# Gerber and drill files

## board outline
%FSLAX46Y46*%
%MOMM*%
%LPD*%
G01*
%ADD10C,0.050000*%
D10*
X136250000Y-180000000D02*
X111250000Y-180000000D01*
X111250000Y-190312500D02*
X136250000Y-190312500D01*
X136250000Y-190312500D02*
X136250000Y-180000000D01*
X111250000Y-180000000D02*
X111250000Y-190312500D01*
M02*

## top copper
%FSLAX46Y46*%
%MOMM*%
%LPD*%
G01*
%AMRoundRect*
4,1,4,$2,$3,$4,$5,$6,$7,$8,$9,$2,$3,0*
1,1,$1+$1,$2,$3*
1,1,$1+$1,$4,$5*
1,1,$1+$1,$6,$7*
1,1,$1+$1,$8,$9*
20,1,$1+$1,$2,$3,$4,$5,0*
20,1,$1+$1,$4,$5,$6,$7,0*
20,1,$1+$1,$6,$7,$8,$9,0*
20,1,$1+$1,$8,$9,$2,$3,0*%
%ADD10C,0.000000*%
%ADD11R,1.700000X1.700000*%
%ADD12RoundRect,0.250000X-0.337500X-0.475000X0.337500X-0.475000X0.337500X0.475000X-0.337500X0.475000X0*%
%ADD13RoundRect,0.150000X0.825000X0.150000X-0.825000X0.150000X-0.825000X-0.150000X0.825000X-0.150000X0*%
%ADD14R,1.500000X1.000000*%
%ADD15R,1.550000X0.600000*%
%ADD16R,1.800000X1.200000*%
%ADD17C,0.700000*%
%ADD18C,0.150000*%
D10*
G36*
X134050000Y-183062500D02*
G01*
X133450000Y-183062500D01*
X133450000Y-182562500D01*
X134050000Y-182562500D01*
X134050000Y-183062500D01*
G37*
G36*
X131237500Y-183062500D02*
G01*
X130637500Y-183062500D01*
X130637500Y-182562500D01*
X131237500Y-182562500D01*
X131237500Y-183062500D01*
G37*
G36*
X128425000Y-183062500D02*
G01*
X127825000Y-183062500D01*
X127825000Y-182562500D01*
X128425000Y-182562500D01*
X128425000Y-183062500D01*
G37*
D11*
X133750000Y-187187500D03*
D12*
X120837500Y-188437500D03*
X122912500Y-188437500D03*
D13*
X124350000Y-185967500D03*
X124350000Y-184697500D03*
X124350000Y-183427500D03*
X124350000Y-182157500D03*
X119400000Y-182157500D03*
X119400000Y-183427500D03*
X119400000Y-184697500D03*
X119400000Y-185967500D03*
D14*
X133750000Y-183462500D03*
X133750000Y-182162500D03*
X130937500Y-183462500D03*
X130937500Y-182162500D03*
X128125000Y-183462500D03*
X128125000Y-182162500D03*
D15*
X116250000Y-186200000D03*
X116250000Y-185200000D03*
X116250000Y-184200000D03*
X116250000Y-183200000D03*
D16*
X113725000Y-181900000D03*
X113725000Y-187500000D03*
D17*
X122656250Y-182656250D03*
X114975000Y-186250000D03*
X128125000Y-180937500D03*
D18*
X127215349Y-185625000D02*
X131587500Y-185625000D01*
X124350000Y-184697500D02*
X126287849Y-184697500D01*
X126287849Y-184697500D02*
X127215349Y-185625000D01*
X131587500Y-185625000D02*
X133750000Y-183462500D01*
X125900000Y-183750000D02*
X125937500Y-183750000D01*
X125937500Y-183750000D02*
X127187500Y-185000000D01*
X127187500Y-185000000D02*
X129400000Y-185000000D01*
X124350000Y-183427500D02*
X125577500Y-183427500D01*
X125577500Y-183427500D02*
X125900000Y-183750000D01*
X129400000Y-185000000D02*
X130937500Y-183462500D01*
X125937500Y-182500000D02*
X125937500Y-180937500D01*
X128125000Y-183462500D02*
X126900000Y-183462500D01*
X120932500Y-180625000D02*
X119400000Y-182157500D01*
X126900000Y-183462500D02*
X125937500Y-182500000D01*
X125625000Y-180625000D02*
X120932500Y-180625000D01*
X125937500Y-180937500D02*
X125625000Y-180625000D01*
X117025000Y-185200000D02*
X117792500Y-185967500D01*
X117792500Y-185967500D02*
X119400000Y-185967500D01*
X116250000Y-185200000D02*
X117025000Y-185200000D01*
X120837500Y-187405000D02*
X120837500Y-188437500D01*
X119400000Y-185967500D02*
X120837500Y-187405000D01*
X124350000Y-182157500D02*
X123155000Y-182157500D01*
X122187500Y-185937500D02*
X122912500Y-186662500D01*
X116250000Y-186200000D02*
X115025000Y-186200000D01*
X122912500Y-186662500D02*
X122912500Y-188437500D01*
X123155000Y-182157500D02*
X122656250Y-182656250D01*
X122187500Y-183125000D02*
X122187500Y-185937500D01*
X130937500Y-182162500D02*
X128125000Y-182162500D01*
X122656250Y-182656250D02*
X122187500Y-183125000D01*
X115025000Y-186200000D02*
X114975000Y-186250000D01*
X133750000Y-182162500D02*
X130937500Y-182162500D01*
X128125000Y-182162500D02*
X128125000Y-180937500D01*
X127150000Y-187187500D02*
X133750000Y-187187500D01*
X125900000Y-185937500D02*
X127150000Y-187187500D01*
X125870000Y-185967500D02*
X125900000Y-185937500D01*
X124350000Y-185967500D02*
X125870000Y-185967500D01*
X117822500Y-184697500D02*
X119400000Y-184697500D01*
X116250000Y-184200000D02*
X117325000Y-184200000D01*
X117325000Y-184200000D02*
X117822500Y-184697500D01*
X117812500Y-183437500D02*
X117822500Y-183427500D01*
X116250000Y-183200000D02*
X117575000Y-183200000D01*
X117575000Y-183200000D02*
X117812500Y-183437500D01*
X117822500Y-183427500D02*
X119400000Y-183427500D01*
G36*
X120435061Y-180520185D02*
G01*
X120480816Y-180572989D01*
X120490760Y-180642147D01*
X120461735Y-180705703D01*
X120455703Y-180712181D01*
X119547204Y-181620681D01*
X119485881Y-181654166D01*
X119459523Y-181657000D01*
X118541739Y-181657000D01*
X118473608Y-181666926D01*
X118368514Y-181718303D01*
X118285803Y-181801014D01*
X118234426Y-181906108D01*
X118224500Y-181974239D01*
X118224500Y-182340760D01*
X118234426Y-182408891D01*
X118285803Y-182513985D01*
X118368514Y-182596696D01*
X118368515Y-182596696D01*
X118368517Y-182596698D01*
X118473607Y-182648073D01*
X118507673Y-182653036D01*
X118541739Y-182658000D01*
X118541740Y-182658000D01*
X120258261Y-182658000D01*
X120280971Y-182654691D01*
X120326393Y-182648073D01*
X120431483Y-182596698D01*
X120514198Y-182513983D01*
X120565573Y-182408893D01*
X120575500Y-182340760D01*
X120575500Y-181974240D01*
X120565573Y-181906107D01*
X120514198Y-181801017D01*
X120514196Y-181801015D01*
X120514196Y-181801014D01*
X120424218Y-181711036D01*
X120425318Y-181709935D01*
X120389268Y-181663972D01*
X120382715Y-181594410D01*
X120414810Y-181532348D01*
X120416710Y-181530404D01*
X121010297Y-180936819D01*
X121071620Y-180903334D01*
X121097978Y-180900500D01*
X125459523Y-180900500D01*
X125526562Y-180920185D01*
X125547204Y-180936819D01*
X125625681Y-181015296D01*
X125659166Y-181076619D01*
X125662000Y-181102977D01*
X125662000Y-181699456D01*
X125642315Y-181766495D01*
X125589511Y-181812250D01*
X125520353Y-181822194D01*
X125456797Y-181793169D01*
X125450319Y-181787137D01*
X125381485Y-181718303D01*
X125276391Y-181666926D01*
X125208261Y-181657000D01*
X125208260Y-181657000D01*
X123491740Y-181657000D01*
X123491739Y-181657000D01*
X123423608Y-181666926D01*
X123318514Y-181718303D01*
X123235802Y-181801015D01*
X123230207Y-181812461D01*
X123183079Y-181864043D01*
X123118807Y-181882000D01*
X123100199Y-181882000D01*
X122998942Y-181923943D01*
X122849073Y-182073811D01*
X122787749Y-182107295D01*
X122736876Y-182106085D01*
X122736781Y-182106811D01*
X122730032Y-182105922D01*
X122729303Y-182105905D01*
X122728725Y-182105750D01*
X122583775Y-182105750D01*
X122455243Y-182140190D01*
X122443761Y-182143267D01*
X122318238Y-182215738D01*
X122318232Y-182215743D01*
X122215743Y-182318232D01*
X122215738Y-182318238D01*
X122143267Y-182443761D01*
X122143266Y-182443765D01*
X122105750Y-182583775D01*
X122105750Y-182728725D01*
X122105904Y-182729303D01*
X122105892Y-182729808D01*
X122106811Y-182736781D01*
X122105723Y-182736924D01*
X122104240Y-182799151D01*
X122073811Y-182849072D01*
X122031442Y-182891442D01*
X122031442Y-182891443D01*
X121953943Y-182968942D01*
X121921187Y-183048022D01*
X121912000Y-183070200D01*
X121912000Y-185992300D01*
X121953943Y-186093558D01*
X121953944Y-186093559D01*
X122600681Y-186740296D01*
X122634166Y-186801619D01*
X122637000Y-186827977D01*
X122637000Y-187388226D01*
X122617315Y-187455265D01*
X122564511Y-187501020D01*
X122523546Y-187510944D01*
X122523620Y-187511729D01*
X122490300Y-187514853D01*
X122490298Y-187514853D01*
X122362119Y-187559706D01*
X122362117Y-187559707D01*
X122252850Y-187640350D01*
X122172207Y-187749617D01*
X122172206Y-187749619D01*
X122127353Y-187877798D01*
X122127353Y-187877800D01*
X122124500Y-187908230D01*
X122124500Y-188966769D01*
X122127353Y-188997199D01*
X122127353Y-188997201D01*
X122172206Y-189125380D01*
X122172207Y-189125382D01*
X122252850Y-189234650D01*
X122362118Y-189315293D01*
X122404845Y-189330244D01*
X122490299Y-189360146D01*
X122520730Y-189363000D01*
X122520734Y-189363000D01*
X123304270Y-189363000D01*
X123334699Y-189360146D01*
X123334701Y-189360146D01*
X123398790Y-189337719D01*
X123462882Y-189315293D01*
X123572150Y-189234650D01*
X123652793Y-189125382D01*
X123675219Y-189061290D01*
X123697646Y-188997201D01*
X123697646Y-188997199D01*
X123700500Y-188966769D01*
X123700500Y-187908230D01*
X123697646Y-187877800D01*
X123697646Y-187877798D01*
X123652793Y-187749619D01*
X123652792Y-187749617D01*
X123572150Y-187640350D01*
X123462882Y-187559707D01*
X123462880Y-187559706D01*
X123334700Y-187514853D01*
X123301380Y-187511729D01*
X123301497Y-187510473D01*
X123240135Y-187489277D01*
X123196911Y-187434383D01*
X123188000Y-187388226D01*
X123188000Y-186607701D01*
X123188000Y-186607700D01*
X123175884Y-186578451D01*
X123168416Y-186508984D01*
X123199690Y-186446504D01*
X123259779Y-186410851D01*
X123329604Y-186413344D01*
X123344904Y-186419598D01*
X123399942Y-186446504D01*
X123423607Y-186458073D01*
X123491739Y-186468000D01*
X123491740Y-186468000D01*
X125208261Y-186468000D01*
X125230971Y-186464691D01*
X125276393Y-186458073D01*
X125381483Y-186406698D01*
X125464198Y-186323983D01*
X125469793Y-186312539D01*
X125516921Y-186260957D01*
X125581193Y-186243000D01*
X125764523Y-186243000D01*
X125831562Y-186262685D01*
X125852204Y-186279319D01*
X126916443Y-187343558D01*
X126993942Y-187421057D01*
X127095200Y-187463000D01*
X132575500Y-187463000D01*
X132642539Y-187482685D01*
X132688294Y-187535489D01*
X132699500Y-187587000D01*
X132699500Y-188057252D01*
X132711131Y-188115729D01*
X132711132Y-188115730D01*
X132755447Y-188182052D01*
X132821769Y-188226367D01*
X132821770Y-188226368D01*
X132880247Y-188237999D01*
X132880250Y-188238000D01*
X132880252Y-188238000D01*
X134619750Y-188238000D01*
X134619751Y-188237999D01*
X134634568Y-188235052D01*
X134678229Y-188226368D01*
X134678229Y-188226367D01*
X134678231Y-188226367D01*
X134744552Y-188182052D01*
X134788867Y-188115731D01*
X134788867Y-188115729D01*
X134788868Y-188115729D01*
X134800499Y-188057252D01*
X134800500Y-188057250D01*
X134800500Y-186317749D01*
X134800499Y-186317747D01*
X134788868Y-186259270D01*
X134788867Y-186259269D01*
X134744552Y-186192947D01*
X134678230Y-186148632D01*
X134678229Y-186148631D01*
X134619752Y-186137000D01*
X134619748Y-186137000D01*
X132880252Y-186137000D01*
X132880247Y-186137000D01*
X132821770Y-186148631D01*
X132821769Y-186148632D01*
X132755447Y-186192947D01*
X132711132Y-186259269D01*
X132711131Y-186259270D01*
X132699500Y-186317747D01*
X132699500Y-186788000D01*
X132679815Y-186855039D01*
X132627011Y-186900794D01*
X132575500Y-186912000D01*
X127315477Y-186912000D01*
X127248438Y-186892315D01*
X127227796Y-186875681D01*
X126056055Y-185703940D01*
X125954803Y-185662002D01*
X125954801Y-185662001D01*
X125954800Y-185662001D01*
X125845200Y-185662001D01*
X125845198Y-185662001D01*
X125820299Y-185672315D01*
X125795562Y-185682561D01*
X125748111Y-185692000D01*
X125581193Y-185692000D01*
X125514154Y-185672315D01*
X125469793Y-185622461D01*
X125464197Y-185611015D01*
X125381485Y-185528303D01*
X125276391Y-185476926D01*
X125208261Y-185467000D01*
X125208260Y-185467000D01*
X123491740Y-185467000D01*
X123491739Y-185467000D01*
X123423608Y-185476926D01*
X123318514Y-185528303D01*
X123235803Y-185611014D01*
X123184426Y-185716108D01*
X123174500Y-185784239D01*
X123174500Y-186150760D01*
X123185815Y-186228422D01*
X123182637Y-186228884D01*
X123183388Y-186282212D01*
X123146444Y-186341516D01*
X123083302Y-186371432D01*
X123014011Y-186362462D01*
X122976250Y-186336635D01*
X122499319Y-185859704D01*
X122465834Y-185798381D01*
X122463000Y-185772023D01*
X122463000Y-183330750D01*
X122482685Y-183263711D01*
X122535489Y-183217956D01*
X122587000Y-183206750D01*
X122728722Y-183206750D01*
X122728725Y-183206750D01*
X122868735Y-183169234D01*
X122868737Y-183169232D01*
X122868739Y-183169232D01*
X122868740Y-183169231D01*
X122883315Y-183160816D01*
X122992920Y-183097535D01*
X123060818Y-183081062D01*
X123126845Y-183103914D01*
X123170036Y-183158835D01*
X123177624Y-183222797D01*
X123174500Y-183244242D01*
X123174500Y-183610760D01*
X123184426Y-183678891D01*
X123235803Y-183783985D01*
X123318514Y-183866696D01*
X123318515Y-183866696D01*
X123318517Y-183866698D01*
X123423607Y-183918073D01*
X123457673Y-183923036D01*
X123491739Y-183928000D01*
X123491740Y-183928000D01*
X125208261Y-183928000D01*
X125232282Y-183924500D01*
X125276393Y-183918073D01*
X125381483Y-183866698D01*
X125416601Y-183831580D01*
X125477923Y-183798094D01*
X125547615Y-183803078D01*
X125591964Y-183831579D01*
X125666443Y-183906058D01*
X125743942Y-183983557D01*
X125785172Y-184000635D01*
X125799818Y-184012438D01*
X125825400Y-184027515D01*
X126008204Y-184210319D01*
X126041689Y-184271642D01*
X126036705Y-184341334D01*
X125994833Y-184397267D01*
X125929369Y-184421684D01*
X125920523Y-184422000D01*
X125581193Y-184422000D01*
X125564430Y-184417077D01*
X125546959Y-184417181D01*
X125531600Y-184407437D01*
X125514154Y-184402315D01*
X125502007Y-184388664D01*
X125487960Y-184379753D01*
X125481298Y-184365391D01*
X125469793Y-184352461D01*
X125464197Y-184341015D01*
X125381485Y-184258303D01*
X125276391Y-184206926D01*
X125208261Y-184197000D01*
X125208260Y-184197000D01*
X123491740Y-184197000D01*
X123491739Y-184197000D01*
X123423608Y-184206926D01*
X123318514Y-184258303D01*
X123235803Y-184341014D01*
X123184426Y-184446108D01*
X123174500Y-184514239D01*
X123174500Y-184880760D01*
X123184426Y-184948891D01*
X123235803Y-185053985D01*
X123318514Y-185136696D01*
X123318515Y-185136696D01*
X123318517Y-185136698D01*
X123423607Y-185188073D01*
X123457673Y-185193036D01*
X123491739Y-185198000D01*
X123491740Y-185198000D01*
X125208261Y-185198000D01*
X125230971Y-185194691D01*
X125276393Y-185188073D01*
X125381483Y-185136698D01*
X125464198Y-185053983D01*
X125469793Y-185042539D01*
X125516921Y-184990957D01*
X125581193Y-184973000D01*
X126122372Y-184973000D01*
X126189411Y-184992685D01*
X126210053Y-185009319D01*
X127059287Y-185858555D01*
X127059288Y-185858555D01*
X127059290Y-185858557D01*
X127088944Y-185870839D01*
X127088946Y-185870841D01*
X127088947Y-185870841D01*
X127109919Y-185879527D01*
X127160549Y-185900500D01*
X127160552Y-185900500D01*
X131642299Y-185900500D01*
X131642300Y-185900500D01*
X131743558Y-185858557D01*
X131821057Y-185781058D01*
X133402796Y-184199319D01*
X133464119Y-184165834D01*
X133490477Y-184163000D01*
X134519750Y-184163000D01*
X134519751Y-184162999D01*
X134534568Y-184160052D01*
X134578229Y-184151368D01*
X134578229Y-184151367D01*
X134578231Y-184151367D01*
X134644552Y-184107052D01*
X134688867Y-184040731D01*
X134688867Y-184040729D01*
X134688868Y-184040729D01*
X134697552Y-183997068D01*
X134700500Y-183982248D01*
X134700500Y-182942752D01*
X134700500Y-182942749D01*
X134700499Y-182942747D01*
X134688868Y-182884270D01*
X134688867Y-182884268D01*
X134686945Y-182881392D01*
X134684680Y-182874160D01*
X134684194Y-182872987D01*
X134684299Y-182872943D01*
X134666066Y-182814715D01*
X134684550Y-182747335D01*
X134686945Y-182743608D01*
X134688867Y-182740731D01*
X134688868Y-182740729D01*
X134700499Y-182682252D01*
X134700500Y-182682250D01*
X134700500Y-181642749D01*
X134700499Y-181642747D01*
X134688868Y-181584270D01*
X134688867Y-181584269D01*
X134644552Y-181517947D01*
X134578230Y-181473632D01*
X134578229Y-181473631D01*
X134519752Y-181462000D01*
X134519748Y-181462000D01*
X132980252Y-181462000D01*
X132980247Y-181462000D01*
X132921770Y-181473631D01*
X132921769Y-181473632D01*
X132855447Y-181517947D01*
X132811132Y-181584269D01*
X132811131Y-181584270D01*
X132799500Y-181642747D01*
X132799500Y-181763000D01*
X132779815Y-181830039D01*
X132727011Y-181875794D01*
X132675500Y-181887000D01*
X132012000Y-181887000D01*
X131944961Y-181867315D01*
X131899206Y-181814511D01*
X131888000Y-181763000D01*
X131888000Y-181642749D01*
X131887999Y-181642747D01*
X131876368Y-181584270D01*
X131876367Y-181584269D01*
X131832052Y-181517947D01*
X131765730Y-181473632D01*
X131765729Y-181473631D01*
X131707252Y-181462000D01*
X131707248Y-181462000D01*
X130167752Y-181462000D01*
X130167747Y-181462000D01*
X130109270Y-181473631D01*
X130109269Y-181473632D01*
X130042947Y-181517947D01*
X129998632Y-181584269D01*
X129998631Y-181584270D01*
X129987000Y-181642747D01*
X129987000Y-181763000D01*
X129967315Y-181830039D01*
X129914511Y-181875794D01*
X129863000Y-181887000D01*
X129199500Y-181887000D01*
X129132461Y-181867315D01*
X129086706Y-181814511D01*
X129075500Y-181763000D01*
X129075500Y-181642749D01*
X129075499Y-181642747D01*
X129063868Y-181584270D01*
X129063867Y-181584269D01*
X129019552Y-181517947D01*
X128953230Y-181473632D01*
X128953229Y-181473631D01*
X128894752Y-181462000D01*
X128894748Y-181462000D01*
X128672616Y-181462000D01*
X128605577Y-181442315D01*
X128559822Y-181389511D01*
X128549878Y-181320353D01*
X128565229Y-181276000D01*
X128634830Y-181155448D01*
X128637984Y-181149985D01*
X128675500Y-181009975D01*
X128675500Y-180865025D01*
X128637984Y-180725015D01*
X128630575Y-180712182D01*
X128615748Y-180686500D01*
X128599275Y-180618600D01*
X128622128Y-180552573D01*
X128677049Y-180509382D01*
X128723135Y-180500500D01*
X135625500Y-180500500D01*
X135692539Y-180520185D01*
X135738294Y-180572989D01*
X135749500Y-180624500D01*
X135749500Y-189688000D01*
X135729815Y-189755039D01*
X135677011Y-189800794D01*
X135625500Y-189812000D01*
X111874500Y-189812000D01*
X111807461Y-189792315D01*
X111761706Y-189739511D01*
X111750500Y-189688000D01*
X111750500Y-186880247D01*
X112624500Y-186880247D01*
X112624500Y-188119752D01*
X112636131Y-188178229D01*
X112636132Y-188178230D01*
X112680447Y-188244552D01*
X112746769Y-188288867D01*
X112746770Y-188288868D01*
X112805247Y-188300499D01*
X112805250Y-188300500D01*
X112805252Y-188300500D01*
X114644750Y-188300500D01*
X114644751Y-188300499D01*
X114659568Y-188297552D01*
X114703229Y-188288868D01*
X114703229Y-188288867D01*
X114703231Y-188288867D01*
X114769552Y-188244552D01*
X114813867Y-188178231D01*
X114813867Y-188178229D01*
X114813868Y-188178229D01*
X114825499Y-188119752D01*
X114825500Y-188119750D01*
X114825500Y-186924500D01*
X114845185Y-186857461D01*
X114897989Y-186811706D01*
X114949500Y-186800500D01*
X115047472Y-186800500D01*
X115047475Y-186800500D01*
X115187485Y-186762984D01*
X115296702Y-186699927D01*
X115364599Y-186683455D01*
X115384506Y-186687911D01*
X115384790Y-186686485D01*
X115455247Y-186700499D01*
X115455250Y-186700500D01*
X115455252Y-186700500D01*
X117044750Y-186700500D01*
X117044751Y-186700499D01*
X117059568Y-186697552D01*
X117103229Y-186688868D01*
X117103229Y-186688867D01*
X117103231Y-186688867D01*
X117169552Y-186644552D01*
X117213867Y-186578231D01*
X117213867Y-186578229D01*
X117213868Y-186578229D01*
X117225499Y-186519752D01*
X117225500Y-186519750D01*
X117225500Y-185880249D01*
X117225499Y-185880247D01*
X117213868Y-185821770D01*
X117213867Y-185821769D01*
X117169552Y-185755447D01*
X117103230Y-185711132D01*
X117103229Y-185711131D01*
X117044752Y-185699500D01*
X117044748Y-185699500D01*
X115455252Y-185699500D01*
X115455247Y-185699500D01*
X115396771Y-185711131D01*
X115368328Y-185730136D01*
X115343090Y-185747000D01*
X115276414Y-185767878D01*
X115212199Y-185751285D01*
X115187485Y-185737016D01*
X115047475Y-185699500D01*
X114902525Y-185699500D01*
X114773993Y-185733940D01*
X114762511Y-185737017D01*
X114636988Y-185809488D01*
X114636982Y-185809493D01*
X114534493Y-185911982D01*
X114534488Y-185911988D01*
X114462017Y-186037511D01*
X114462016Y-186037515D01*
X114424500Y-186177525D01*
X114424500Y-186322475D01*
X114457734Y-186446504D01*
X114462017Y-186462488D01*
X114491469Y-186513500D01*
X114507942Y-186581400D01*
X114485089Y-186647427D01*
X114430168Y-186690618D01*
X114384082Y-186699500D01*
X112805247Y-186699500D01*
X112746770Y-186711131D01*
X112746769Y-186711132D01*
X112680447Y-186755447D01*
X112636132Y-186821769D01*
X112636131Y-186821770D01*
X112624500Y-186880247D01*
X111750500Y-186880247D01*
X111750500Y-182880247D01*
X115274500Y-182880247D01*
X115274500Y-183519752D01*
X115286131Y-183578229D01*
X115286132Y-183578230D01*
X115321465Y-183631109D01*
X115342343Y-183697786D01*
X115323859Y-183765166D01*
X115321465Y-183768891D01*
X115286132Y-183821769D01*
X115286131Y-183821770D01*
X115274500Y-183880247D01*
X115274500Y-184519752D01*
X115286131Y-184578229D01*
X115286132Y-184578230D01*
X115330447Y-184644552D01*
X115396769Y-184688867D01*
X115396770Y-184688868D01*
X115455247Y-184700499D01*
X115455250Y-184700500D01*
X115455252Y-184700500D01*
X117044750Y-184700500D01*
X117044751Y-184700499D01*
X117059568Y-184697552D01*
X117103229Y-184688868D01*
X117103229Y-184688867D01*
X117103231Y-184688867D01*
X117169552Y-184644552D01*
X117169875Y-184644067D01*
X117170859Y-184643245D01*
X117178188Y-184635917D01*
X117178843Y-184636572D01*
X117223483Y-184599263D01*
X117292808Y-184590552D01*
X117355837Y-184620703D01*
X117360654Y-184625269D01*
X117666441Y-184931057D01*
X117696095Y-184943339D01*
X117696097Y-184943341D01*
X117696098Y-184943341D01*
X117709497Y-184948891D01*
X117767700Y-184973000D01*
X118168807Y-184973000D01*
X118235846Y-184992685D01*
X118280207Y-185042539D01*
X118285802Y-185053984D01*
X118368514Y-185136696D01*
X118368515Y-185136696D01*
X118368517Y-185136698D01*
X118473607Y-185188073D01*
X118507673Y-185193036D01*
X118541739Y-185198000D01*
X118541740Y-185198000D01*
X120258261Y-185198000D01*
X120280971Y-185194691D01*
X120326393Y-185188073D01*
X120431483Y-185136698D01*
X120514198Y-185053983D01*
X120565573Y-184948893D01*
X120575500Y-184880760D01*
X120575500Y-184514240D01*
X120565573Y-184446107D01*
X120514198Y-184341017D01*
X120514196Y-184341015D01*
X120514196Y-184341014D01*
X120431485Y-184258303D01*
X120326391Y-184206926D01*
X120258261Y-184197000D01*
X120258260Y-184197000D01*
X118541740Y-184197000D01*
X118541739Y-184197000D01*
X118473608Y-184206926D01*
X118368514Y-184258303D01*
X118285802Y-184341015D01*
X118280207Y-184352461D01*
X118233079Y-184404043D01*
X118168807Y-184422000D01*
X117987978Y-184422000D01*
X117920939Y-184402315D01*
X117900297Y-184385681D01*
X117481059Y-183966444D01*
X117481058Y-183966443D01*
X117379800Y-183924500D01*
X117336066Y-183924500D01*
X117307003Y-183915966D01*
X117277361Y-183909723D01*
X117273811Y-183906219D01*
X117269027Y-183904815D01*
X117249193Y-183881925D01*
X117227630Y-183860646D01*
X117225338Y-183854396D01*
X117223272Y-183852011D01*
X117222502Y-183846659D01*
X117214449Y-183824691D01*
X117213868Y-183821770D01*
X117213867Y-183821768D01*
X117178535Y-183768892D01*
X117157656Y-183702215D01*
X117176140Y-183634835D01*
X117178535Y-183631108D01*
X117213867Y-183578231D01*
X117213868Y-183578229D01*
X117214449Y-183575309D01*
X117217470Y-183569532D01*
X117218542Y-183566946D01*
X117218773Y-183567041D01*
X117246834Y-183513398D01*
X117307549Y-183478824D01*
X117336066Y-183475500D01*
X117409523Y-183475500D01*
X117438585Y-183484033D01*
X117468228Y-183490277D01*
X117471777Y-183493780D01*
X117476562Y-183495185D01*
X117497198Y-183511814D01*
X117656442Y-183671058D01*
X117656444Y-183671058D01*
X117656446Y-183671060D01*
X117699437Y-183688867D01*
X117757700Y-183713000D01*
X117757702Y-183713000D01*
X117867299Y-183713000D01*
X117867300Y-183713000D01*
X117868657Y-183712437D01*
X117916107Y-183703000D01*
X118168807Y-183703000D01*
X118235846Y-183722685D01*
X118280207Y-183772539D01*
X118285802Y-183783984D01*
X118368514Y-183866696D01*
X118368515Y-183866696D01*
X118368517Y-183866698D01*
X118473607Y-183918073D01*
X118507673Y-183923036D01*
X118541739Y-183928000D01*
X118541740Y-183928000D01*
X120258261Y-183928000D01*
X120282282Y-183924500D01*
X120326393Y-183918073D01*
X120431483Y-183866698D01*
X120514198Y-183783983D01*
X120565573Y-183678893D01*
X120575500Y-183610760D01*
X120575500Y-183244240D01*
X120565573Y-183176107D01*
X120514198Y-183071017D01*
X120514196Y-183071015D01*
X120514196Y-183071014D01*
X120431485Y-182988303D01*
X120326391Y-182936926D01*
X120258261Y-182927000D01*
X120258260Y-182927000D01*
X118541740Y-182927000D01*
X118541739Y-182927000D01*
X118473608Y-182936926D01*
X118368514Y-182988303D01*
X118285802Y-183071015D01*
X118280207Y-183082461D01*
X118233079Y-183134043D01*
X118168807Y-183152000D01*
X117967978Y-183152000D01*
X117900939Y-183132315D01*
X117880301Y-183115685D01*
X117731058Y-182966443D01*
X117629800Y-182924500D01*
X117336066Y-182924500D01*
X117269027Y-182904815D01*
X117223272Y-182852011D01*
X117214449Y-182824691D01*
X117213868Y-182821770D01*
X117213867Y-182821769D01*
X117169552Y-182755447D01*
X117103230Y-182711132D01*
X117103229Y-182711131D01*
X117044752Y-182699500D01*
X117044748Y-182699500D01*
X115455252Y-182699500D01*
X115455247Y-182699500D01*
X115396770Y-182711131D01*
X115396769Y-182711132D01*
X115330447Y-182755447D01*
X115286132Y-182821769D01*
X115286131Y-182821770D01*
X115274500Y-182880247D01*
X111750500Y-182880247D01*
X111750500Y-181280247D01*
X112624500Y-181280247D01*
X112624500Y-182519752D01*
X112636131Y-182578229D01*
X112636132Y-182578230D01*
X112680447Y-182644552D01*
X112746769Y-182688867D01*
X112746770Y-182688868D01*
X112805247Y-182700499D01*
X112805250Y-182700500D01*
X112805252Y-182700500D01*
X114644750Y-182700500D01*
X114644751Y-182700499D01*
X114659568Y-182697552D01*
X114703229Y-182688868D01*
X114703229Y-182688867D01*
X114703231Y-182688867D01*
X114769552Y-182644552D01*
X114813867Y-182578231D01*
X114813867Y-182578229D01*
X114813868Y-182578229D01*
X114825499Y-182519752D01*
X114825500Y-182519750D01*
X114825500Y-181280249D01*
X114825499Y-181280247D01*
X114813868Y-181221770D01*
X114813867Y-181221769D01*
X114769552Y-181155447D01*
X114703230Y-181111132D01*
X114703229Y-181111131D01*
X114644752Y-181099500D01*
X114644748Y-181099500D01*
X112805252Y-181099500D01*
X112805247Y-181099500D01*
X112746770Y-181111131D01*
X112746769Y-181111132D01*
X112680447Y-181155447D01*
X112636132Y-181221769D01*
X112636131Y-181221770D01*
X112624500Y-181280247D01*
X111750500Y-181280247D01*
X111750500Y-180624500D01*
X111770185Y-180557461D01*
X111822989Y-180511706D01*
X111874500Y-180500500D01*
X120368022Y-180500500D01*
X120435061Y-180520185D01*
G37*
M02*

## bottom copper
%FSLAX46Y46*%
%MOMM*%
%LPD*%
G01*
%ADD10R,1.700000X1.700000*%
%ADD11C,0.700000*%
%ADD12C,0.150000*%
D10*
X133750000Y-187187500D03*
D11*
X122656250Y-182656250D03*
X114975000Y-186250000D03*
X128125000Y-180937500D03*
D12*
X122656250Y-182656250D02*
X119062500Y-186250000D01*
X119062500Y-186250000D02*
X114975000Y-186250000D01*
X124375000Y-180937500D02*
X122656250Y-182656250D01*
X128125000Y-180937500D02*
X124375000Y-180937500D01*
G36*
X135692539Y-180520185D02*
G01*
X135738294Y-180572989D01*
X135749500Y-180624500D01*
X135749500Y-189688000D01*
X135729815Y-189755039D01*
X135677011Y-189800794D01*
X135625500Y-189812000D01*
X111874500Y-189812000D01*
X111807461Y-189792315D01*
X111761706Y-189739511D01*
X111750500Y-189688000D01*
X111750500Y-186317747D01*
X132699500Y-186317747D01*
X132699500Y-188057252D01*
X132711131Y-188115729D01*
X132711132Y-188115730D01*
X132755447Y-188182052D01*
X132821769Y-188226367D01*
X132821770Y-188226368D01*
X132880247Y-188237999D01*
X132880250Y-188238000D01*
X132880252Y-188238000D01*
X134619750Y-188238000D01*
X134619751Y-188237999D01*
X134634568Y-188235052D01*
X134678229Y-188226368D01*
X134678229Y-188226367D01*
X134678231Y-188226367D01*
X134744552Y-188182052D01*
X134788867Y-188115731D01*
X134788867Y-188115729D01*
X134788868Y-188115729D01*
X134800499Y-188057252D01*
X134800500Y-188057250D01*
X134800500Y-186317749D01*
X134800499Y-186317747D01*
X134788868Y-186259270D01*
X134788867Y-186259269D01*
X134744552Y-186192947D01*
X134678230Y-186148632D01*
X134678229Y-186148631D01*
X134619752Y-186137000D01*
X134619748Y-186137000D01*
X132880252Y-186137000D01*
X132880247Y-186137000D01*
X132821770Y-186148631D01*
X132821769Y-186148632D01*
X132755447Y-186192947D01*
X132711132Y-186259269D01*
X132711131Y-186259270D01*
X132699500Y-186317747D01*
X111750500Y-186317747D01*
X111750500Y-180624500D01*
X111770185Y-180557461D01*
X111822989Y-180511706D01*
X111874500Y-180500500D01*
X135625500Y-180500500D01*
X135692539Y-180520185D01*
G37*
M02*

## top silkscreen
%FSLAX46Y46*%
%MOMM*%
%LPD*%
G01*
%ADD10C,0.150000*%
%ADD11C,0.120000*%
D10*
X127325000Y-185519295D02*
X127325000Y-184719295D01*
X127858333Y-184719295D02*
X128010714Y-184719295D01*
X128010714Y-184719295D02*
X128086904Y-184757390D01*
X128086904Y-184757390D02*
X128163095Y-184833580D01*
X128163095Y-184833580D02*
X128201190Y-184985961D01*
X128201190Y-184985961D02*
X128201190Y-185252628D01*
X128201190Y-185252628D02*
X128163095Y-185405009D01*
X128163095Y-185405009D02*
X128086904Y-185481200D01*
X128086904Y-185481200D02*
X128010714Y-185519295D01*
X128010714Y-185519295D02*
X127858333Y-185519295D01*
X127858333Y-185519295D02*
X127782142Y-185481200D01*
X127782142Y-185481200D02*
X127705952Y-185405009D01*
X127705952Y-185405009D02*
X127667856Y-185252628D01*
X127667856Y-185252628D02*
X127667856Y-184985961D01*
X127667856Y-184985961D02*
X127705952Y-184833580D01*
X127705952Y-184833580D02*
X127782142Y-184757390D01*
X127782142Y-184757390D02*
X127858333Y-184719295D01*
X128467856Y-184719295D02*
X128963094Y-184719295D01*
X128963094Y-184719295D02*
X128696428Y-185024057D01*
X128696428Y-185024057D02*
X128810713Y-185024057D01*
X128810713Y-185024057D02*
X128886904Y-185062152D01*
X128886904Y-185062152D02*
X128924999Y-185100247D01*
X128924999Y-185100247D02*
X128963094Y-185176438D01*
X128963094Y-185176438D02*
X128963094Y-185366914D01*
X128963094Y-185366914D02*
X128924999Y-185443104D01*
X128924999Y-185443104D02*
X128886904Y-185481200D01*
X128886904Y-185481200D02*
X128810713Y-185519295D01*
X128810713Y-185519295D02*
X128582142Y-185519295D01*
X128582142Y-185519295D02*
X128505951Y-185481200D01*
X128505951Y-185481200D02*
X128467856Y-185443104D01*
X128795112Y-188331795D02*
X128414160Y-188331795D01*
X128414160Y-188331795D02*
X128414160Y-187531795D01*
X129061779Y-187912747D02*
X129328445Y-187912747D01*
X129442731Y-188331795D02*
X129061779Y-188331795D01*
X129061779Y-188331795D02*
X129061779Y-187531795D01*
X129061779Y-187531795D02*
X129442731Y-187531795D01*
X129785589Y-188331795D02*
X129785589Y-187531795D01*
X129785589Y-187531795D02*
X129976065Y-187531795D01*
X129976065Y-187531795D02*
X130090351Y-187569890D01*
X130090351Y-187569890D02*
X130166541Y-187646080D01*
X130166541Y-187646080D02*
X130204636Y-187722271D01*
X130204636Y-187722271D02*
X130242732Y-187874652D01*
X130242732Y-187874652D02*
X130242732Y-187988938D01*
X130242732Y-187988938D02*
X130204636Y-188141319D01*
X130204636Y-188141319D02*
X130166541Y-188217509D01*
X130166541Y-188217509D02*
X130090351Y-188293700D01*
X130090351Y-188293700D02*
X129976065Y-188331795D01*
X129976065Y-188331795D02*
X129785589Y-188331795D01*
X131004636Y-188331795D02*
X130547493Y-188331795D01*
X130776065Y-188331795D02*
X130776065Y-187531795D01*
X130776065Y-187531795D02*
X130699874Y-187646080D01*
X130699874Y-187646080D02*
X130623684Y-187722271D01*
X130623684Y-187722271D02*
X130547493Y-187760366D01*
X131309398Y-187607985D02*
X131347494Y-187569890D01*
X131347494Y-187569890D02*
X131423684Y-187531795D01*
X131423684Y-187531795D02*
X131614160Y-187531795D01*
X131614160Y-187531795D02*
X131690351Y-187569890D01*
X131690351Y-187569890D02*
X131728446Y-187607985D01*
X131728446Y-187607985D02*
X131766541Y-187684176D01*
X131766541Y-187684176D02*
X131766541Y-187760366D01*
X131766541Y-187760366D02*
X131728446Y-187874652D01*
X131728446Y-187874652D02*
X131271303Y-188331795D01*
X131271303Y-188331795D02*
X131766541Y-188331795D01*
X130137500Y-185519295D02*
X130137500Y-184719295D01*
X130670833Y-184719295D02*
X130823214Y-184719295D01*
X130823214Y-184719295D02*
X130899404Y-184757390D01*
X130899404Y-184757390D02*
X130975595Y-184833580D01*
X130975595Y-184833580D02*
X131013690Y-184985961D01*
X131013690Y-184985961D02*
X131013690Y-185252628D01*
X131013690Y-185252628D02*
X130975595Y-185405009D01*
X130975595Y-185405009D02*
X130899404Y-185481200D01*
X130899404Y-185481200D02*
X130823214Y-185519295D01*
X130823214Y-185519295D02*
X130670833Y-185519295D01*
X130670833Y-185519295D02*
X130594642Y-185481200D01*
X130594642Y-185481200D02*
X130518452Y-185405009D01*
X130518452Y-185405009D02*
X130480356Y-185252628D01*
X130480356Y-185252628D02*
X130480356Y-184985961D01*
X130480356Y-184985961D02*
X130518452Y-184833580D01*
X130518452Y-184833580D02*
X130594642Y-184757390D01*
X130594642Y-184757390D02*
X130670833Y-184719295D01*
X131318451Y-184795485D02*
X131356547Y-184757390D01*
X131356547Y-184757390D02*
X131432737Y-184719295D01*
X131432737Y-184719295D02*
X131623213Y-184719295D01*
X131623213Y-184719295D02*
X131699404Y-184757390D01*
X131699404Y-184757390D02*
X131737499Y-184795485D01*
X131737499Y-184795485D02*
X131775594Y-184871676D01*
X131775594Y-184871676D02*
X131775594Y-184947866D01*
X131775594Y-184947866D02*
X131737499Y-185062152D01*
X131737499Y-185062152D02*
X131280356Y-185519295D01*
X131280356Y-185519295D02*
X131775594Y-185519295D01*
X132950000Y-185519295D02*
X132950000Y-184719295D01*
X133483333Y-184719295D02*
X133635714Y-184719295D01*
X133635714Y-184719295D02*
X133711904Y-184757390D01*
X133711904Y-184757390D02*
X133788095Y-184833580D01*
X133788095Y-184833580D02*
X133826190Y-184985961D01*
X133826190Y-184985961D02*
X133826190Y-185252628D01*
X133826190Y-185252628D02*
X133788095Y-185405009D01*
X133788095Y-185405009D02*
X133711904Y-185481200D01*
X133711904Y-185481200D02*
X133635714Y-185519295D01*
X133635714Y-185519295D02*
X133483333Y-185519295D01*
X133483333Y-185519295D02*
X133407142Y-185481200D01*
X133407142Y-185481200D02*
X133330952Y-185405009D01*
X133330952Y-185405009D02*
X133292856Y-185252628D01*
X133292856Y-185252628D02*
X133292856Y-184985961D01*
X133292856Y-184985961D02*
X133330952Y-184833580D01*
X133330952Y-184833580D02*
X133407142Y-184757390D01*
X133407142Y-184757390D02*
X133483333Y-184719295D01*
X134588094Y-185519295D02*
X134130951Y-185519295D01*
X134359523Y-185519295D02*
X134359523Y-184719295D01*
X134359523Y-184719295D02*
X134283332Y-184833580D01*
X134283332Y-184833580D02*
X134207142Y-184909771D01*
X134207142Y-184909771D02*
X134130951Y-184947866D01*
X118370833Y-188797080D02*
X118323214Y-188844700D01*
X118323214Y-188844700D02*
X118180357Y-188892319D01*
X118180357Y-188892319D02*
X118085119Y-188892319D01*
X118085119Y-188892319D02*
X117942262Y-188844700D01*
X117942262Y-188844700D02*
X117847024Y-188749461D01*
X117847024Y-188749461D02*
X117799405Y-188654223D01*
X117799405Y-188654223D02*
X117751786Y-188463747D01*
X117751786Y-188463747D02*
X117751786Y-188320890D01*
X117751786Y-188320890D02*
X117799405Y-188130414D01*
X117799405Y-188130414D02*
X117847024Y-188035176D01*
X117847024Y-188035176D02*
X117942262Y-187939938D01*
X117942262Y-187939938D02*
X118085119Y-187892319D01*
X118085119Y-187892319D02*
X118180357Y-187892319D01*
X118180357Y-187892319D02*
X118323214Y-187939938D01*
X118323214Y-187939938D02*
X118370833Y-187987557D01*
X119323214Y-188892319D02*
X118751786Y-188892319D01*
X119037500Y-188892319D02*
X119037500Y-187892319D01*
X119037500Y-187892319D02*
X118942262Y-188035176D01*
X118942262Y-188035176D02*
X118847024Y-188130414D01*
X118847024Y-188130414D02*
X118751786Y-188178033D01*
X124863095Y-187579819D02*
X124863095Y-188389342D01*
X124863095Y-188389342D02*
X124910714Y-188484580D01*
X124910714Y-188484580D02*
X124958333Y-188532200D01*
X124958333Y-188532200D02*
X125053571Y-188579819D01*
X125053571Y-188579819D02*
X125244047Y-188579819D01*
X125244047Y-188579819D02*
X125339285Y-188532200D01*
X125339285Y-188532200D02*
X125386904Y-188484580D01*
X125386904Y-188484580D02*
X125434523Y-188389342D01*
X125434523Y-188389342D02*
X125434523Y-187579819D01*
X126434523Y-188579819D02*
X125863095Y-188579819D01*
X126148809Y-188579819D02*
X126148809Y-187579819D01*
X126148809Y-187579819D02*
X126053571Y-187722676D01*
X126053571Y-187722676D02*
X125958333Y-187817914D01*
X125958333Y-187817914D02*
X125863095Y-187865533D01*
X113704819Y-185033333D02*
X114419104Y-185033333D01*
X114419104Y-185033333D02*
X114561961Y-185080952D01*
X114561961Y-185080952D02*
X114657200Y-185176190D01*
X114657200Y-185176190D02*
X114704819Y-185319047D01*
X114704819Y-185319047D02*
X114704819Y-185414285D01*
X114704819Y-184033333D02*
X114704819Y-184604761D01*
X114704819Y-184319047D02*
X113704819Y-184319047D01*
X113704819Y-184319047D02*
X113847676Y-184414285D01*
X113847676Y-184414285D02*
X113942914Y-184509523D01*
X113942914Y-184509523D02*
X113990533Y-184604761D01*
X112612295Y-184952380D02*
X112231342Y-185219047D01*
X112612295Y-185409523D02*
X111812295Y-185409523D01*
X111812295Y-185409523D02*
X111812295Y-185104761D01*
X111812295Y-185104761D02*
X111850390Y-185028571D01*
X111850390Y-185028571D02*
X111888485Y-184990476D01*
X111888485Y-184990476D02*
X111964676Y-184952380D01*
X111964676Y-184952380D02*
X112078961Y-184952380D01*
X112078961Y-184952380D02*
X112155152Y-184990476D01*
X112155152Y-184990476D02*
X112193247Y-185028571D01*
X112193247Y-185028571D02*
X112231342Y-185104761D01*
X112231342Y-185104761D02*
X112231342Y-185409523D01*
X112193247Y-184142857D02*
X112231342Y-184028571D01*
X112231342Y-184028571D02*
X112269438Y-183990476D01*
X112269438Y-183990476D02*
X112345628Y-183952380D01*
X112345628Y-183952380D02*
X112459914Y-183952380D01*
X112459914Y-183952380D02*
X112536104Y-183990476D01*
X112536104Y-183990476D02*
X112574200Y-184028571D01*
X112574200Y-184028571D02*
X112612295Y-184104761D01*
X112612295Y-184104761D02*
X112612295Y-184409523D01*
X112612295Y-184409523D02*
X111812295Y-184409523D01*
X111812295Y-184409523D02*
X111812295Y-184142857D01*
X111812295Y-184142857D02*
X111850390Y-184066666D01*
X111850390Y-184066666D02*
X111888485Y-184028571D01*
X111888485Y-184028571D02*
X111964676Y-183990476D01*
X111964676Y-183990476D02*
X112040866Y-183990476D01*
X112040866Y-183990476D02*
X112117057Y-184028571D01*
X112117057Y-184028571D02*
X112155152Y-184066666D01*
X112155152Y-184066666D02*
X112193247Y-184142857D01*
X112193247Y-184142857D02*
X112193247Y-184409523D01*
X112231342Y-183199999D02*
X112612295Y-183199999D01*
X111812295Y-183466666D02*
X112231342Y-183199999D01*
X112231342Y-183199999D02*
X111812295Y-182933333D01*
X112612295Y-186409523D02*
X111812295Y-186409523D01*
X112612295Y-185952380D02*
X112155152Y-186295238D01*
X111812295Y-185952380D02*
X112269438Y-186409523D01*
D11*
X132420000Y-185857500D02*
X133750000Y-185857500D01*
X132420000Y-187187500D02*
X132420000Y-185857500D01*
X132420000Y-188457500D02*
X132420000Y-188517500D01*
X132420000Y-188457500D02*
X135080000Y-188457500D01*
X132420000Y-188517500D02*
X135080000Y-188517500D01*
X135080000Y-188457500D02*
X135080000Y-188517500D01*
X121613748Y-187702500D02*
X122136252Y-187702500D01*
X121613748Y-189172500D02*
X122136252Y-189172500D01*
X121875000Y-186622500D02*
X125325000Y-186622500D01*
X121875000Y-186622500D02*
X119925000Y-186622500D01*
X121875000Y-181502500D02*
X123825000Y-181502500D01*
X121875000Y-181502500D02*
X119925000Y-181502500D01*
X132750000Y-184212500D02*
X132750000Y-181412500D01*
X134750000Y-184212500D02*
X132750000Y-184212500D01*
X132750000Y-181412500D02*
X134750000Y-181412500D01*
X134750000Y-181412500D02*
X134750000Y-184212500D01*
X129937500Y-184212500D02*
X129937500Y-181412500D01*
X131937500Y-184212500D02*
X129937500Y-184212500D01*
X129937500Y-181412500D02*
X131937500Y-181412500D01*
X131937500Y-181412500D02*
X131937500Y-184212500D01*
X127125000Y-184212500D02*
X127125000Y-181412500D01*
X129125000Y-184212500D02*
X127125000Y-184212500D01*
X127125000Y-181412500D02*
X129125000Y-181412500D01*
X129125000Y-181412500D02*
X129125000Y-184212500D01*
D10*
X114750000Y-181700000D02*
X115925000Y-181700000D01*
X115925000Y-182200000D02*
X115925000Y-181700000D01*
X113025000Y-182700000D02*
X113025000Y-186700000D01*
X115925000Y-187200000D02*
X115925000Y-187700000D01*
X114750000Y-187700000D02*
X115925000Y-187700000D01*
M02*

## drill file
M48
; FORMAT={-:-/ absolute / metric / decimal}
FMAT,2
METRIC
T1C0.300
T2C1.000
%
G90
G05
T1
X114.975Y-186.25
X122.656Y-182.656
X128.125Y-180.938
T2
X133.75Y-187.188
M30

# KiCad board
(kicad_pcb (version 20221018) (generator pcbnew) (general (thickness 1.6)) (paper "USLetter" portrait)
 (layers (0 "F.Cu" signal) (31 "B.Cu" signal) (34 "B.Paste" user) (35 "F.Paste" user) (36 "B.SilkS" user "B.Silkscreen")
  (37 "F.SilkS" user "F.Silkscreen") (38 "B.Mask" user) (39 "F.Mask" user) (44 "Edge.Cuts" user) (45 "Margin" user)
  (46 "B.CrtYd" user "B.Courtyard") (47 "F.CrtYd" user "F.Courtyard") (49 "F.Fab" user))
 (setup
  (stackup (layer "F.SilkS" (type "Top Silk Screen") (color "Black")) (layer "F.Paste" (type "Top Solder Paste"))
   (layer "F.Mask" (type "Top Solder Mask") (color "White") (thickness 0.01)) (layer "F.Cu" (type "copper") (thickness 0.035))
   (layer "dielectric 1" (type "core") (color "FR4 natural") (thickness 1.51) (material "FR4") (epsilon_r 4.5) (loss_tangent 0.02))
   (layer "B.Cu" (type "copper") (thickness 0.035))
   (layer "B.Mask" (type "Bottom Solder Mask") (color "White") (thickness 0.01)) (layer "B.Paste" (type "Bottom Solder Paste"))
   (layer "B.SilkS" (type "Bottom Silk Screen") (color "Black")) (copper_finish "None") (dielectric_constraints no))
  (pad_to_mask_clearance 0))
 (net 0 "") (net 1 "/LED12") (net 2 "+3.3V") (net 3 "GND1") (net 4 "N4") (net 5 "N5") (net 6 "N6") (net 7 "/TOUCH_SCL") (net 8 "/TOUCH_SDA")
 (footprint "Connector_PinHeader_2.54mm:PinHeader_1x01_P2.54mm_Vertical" (layer "F.Cu") (at 133.75 187.1875)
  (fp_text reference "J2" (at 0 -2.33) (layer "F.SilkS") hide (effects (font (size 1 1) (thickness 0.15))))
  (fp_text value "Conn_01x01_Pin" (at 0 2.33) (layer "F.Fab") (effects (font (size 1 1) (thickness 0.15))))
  (fp_line (start -1.33 -1.33) (end 0 -1.33) (stroke (width 0.12) (type solid)) (layer "F.SilkS"))
  (fp_line (start -1.33 0) (end -1.33 -1.33) (stroke (width 0.12) (type solid)) (layer "F.SilkS"))
  (fp_line (start -1.33 1.27) (end -1.33 1.33) (stroke (width 0.12) (type solid)) (layer "F.SilkS"))
  (fp_line (start -1.33 1.27) (end 1.33 1.27) (stroke (width 0.12) (type solid)) (layer "F.SilkS"))
  (fp_line (start -1.33 1.33) (end 1.33 1.33) (stroke (width 0.12) (type solid)) (layer "F.SilkS"))
  (fp_line (start 1.33 1.27) (end 1.33 1.33) (stroke (width 0.12) (type solid)) (layer "F.SilkS"))
  (pad "1" thru_hole rect (at 0 0) (size 1.7 1.7) (drill 1) (layers "*.Cu" "*.Mask") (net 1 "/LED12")))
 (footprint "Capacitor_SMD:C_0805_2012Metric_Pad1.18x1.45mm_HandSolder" (layer "F.Cu") (at 121.875 188.4375)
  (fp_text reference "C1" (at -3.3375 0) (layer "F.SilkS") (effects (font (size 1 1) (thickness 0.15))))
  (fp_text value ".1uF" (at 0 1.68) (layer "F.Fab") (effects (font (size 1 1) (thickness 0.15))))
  (fp_line (start -0.261252 -0.735) (end 0.261252 -0.735) (stroke (width 0.12) (type solid)) (layer "F.SilkS"))
  (fp_line (start -0.261252 0.735) (end 0.261252 0.735) (stroke (width 0.12) (type solid)) (layer "F.SilkS"))
  (pad "1" smd roundrect (at -1.0375 0) (size 1.175 1.45) (layers "F.Cu" "F.Paste" "F.Mask") (roundrect_rratio 0.2127659574) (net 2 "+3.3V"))
  (pad "2" smd roundrect (at 1.0375 0) (size 1.175 1.45) (layers "F.Cu" "F.Paste" "F.Mask") (roundrect_rratio 0.2127659574) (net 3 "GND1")))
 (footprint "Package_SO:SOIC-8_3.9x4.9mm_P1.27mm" (layer "F.Cu") (at 121.875 184.0625 180)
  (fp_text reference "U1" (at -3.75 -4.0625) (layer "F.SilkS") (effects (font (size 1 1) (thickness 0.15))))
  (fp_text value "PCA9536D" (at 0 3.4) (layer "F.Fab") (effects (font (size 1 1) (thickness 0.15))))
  (fp_line (start 0 -2.56) (end -3.45 -2.56) (stroke (width 0.12) (type solid)) (layer "F.SilkS"))
  (fp_line (start 0 -2.56) (end 1.95 -2.56) (stroke (width 0.12) (type solid)) (layer "F.SilkS"))
  (fp_line (start 0 2.56) (end -1.95 2.56) (stroke (width 0.12) (type solid)) (layer "F.SilkS"))
  (fp_line (start 0 2.56) (end 1.95 2.56) (stroke (width 0.12) (type solid)) (layer "F.SilkS"))
  (pad "1" smd roundrect (at -2.475 -1.905 180) (size 1.95 0.6) (layers "F.Cu" "F.Paste" "F.Mask") (roundrect_rratio 0.25) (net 1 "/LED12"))
  (pad "2" smd roundrect (at -2.475 -0.635 180) (size 1.95 0.6) (layers "F.Cu" "F.Paste" "F.Mask") (roundrect_rratio 0.25) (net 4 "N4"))
  (pad "3" smd roundrect (at -2.475 0.635 180) (size 1.95 0.6) (layers "F.Cu" "F.Paste" "F.Mask") (roundrect_rratio 0.25) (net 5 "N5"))
  (pad "4" smd roundrect (at -2.475 1.905 180) (size 1.95 0.6) (layers "F.Cu" "F.Paste" "F.Mask") (roundrect_rratio 0.25) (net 3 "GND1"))
  (pad "5" smd roundrect (at 2.475 1.905 180) (size 1.95 0.6) (layers "F.Cu" "F.Paste" "F.Mask") (roundrect_rratio 0.25) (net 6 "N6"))
  (pad "6" smd roundrect (at 2.475 0.635 180) (size 1.95 0.6) (layers "F.Cu" "F.Paste" "F.Mask") (roundrect_rratio 0.25)
   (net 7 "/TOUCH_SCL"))
  (pad "7" smd roundrect (at 2.475 -0.635 180) (size 1.95 0.6) (layers "F.Cu" "F.Paste" "F.Mask") (roundrect_rratio 0.25)
   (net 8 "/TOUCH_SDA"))
  (pad "8" smd roundrect (at 2.475 -1.905 180) (size 1.95 0.6) (layers "F.Cu" "F.Paste" "F.Mask") (roundrect_rratio 0.25) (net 2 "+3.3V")))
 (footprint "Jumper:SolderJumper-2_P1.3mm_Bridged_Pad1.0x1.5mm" (layer "F.Cu") (at 133.75 182.8125 90) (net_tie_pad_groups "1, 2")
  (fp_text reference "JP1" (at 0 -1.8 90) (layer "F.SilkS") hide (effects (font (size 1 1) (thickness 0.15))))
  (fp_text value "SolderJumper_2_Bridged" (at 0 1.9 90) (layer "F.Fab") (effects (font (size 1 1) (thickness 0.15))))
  (fp_poly (pts (xy -0.25 -0.3) (xy 0.25 -0.3) (xy 0.25 0.3) (xy -0.25 0.3)) (stroke (width 0) (type solid)) (fill solid) (layer "F.Cu"))
  (fp_line (start -1.4 -1) (end 1.4 -1) (stroke (width 0.12) (type solid)) (layer "F.SilkS"))
  (fp_line (start -1.4 1) (end -1.4 -1) (stroke (width 0.12) (type solid)) (layer "F.SilkS"))
  (fp_line (start 1.4 -1) (end 1.4 1) (stroke (width 0.12) (type solid)) (layer "F.SilkS"))
  (fp_line (start 1.4 1) (end -1.4 1) (stroke (width 0.12) (type solid)) (layer "F.SilkS"))
  (pad "1" smd rect (at -0.65 0 90) (size 1 1.5) (layers "F.Cu" "F.Mask") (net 4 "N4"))
  (pad "2" smd rect (at 0.65 0 90) (size 1 1.5) (layers "F.Cu" "F.Mask") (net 3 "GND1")))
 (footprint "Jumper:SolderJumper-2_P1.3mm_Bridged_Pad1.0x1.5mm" (layer "F.Cu") (at 130.9375 182.8125 90) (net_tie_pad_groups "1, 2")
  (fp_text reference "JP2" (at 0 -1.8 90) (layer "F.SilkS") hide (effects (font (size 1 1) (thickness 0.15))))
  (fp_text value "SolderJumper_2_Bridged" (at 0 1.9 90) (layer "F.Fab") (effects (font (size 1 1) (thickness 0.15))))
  (fp_poly (pts (xy -0.25 -0.3) (xy 0.25 -0.3) (xy 0.25 0.3) (xy -0.25 0.3)) (stroke (width 0) (type solid)) (fill solid) (layer "F.Cu"))
  (fp_line (start -1.4 -1) (end 1.4 -1) (stroke (width 0.12) (type solid)) (layer "F.SilkS"))
  (fp_line (start -1.4 1) (end -1.4 -1) (stroke (width 0.12) (type solid)) (layer "F.SilkS"))
  (fp_line (start 1.4 -1) (end 1.4 1) (stroke (width 0.12) (type solid)) (layer "F.SilkS"))
  (fp_line (start 1.4 1) (end -1.4 1) (stroke (width 0.12) (type solid)) (layer "F.SilkS"))
  (pad "1" smd rect (at -0.65 0 90) (size 1 1.5) (layers "F.Cu" "F.Mask") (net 5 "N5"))
  (pad "2" smd rect (at 0.65 0 90) (size 1 1.5) (layers "F.Cu" "F.Mask") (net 3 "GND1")))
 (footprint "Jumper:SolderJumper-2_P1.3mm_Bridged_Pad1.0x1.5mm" (layer "F.Cu") (at 128.125 182.8125 90) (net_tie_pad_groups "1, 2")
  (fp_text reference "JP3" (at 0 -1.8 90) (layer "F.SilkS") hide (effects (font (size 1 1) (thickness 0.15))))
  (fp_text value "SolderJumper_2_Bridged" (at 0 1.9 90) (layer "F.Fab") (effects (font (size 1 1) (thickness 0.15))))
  (fp_poly (pts (xy -0.25 -0.3) (xy 0.25 -0.3) (xy 0.25 0.3) (xy -0.25 0.3)) (stroke (width 0) (type solid)) (fill solid) (layer "F.Cu"))
  (fp_line (start -1.4 -1) (end 1.4 -1) (stroke (width 0.12) (type solid)) (layer "F.SilkS"))
  (fp_line (start -1.4 1) (end -1.4 -1) (stroke (width 0.12) (type solid)) (layer "F.SilkS"))
  (fp_line (start 1.4 -1) (end 1.4 1) (stroke (width 0.12) (type solid)) (layer "F.SilkS"))
  (fp_line (start 1.4 1) (end -1.4 1) (stroke (width 0.12) (type solid)) (layer "F.SilkS"))
  (pad "1" smd rect (at -0.65 0 90) (size 1 1.5) (layers "F.Cu" "F.Mask") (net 6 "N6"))
  (pad "2" smd rect (at 0.65 0 90) (size 1 1.5) (layers "F.Cu" "F.Mask") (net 3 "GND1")))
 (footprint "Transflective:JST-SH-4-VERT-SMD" (layer "F.Cu") (at 116.25 184.7 -90)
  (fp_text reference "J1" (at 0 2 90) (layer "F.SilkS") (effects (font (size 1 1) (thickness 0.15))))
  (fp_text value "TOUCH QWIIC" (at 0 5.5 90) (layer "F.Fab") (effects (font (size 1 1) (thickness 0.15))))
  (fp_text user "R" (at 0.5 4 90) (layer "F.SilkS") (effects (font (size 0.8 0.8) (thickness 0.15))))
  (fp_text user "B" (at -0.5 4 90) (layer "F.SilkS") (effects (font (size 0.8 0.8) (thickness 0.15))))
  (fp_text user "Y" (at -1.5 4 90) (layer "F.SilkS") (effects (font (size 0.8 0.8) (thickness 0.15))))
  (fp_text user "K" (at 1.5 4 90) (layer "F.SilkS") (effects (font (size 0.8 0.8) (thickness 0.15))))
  (fp_line (start -3 1.5) (end -3 0.325) (stroke (width 0.15) (type solid)) (layer "F.SilkS"))
  (fp_line (start -2.5 0.325) (end -3 0.325) (stroke (width 0.15) (type solid)) (layer "F.SilkS"))
  (fp_line (start -2 3.225) (end 2 3.225) (stroke (width 0.15) (type solid)) (layer "F.SilkS"))
  (fp_line (start 2.5 0.325) (end 3 0.325) (stroke (width 0.15) (type solid)) (layer "F.SilkS"))
  (fp_line (start 3 1.5) (end 3 0.325) (stroke (width 0.15) (type solid)) (layer "F.SilkS"))
  (pad "1" smd rect (at 1.5 0 270) (size 0.6 1.55) (layers "F.Cu" "F.Paste" "F.Mask") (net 3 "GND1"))
  (pad "2" smd rect (at 0.5 0 270) (size 0.6 1.55) (layers "F.Cu" "F.Paste" "F.Mask") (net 2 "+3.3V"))
  (pad "3" smd rect (at -0.5 0 270) (size 0.6 1.55) (layers "F.Cu" "F.Paste" "F.Mask") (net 8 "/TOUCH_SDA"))
  (pad "4" smd rect (at -1.5 0 270) (size 0.6 1.55) (layers "F.Cu" "F.Paste" "F.Mask") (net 7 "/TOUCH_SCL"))
  (pad "M" smd rect (at -2.8 2.525 270) (size 1.2 1.8) (layers "F.Cu" "F.Paste" "F.Mask"))
  (pad "M" smd rect (at 2.8 2.525 270) (size 1.2 1.8) (layers "F.Cu" "F.Paste" "F.Mask")))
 (gr_line (start 136.25 180) (end 111.25 180) (stroke (width 0.05) (type default)) (layer "Edge.Cuts"))
 (gr_line (start 111.25 190.3125) (end 136.25 190.3125) (stroke (width 0.05) (type default)) (layer "Edge.Cuts"))
 (gr_line (start 136.25 190.3125) (end 136.25 180) (stroke (width 0.05) (type default)) (layer "Edge.Cuts"))
 (gr_line (start 111.25 180) (end 111.25 190.3125) (stroke (width 0.05) (type default)) (layer "Edge.Cuts"))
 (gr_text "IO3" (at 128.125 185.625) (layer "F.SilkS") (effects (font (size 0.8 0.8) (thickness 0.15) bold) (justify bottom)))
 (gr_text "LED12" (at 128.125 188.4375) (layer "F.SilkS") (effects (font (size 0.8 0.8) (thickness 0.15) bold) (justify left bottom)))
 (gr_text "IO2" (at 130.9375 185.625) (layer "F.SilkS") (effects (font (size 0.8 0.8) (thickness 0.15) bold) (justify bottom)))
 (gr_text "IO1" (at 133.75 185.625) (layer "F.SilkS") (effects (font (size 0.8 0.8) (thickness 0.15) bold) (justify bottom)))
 (segment (start 127.215349 185.625) (end 131.5875 185.625) (width 0.15) (layer "F.Cu") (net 4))
 (segment (start 124.35 184.6975) (end 126.287849 184.6975) (width 0.15) (layer "F.Cu") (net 4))
 (segment (start 126.287849 184.6975) (end 127.215349 185.625) (width 0.15) (layer "F.Cu") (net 4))
 (segment (start 131.5875 185.625) (end 133.75 183.4625) (width 0.15) (layer "F.Cu") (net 4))
 (segment (start 125.9 183.75) (end 125.9375 183.75) (width 0.15) (layer "F.Cu") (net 5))
 (segment (start 125.9375 183.75) (end 127.1875 185) (width 0.15) (layer "F.Cu") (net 5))
 (segment (start 127.1875 185) (end 129.4 185) (width 0.15) (layer "F.Cu") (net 5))
 (segment (start 124.35 183.4275) (end 125.5775 183.4275) (width 0.15) (layer "F.Cu") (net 5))
 (segment (start 125.5775 183.4275) (end 125.9 183.75) (width 0.15) (layer "F.Cu") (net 5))
 (segment (start 129.4 185) (end 130.9375 183.4625) (width 0.15) (layer "F.Cu") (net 5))
 (segment (start 125.9375 182.5) (end 125.9375 180.9375) (width 0.15) (layer "F.Cu") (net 6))
 (segment (start 128.125 183.4625) (end 126.9 183.4625) (width 0.15) (layer "F.Cu") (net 6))
 (segment (start 120.9325 180.625) (end 119.4 182.1575) (width 0.15) (layer "F.Cu") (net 6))
 (segment (start 126.9 183.4625) (end 125.9375 182.5) (width 0.15) (layer "F.Cu") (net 6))
 (segment (start 125.625 180.625) (end 120.9325 180.625) (width 0.15) (layer "F.Cu") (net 6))
 (segment (start 125.9375 180.9375) (end 125.625 180.625) (width 0.15) (layer "F.Cu") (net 6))
 (segment (start 117.025 185.2) (end 117.7925 185.9675) (width 0.15) (layer "F.Cu") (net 2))
 (segment (start 117.7925 185.9675) (end 119.4 185.9675) (width 0.15) (layer "F.Cu") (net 2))
 (segment (start 116.25 185.2) (end 117.025 185.2) (width 0.15) (layer "F.Cu") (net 2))
 (segment (start 120.8375 187.405) (end 120.8375 188.4375) (width 0.15) (layer "F.Cu") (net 2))
 (segment (start 119.4 185.9675) (end 120.8375 187.405) (width 0.15) (layer "F.Cu") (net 2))
 (segment (start 124.35 182.1575) (end 123.155 182.1575) (width 0.15) (layer "F.Cu") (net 3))
 (segment (start 122.1875 185.9375) (end 122.9125 186.6625) (width 0.15) (layer "F.Cu") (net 3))
 (segment (start 116.25 186.2) (end 115.025 186.2) (width 0.15) (layer "F.Cu") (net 3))
 (segment (start 122.9125 186.6625) (end 122.9125 188.4375) (width 0.15) (layer "F.Cu") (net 3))
 (segment (start 123.155 182.1575) (end 122.65625 182.65625) (width 0.15) (layer "F.Cu") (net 3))
 (segment (start 122.1875 183.125) (end 122.1875 185.9375) (width 0.15) (layer "F.Cu") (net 3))
 (segment (start 130.9375 182.1625) (end 128.125 182.1625) (width 0.15) (layer "F.Cu") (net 3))
 (segment (start 122.65625 182.65625) (end 122.1875 183.125) (width 0.15) (layer "F.Cu") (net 3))
 (segment (start 115.025 186.2) (end 114.975 186.25) (width 0.15) (layer "F.Cu") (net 3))
 (segment (start 133.75 182.1625) (end 130.9375 182.1625) (width 0.15) (layer "F.Cu") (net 3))
 (segment (start 128.125 182.1625) (end 128.125 180.9375) (width 0.15) (layer "F.Cu") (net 3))
 (via (at 122.65625 182.65625) (size 0.7) (drill 0.3) (layers "F.Cu" "B.Cu") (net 3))
 (via (at 114.975 186.25) (size 0.7) (drill 0.3) (layers "F.Cu" "B.Cu") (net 3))
 (via (at 128.125 180.9375) (size 0.7) (drill 0.3) (layers "F.Cu" "B.Cu") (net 3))
 (segment (start 122.65625 182.65625) (end 119.0625 186.25) (width 0.15) (layer "B.Cu") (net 3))
 (segment (start 119.0625 186.25) (end 114.975 186.25) (width 0.15) (layer "B.Cu") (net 3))
 (segment (start 124.375 180.9375) (end 122.65625 182.65625) (width 0.15) (layer "B.Cu") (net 3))
 (segment (start 128.125 180.9375) (end 124.375 180.9375) (width 0.15) (layer "B.Cu") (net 3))
 (segment (start 127.15 187.1875) (end 133.75 187.1875) (width 0.15) (layer "F.Cu") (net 1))
 (segment (start 125.9 185.9375) (end 127.15 187.1875) (width 0.15) (layer "F.Cu") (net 1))
 (segment (start 125.87 185.9675) (end 125.9 185.9375) (width 0.15) (layer "F.Cu") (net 1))
 (segment (start 124.35 185.9675) (end 125.87 185.9675) (width 0.15) (layer "F.Cu") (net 1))
 (segment (start 117.8225 184.6975) (end 119.4 184.6975) (width 0.15) (layer "F.Cu") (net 8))
 (segment (start 116.25 184.2) (end 117.325 184.2) (width 0.15) (layer "F.Cu") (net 8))
 (segment (start 117.325 184.2) (end 117.8225 184.6975) (width 0.15) (layer "F.Cu") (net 8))
 (segment (start 117.8125 183.4375) (end 117.8225 183.4275) (width 0.15) (layer "F.Cu") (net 7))
 (segment (start 116.25 183.2) (end 117.575 183.2) (width 0.15) (layer "F.Cu") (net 7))
 (segment (start 117.575 183.2) (end 117.8125 183.4375) (width 0.15) (layer "F.Cu") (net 7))
 (segment (start 117.8225 183.4275) (end 119.4 183.4275) (width 0.15) (layer "F.Cu") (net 7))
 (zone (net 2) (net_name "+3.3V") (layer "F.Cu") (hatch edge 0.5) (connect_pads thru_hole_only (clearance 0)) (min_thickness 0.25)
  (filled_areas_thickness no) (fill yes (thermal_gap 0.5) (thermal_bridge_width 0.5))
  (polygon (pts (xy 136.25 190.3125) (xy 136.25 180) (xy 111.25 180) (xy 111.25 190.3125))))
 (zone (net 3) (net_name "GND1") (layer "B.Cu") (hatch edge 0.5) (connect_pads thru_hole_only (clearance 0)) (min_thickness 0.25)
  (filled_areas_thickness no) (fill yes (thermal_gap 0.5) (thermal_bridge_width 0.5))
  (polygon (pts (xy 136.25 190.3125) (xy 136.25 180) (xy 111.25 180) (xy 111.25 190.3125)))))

